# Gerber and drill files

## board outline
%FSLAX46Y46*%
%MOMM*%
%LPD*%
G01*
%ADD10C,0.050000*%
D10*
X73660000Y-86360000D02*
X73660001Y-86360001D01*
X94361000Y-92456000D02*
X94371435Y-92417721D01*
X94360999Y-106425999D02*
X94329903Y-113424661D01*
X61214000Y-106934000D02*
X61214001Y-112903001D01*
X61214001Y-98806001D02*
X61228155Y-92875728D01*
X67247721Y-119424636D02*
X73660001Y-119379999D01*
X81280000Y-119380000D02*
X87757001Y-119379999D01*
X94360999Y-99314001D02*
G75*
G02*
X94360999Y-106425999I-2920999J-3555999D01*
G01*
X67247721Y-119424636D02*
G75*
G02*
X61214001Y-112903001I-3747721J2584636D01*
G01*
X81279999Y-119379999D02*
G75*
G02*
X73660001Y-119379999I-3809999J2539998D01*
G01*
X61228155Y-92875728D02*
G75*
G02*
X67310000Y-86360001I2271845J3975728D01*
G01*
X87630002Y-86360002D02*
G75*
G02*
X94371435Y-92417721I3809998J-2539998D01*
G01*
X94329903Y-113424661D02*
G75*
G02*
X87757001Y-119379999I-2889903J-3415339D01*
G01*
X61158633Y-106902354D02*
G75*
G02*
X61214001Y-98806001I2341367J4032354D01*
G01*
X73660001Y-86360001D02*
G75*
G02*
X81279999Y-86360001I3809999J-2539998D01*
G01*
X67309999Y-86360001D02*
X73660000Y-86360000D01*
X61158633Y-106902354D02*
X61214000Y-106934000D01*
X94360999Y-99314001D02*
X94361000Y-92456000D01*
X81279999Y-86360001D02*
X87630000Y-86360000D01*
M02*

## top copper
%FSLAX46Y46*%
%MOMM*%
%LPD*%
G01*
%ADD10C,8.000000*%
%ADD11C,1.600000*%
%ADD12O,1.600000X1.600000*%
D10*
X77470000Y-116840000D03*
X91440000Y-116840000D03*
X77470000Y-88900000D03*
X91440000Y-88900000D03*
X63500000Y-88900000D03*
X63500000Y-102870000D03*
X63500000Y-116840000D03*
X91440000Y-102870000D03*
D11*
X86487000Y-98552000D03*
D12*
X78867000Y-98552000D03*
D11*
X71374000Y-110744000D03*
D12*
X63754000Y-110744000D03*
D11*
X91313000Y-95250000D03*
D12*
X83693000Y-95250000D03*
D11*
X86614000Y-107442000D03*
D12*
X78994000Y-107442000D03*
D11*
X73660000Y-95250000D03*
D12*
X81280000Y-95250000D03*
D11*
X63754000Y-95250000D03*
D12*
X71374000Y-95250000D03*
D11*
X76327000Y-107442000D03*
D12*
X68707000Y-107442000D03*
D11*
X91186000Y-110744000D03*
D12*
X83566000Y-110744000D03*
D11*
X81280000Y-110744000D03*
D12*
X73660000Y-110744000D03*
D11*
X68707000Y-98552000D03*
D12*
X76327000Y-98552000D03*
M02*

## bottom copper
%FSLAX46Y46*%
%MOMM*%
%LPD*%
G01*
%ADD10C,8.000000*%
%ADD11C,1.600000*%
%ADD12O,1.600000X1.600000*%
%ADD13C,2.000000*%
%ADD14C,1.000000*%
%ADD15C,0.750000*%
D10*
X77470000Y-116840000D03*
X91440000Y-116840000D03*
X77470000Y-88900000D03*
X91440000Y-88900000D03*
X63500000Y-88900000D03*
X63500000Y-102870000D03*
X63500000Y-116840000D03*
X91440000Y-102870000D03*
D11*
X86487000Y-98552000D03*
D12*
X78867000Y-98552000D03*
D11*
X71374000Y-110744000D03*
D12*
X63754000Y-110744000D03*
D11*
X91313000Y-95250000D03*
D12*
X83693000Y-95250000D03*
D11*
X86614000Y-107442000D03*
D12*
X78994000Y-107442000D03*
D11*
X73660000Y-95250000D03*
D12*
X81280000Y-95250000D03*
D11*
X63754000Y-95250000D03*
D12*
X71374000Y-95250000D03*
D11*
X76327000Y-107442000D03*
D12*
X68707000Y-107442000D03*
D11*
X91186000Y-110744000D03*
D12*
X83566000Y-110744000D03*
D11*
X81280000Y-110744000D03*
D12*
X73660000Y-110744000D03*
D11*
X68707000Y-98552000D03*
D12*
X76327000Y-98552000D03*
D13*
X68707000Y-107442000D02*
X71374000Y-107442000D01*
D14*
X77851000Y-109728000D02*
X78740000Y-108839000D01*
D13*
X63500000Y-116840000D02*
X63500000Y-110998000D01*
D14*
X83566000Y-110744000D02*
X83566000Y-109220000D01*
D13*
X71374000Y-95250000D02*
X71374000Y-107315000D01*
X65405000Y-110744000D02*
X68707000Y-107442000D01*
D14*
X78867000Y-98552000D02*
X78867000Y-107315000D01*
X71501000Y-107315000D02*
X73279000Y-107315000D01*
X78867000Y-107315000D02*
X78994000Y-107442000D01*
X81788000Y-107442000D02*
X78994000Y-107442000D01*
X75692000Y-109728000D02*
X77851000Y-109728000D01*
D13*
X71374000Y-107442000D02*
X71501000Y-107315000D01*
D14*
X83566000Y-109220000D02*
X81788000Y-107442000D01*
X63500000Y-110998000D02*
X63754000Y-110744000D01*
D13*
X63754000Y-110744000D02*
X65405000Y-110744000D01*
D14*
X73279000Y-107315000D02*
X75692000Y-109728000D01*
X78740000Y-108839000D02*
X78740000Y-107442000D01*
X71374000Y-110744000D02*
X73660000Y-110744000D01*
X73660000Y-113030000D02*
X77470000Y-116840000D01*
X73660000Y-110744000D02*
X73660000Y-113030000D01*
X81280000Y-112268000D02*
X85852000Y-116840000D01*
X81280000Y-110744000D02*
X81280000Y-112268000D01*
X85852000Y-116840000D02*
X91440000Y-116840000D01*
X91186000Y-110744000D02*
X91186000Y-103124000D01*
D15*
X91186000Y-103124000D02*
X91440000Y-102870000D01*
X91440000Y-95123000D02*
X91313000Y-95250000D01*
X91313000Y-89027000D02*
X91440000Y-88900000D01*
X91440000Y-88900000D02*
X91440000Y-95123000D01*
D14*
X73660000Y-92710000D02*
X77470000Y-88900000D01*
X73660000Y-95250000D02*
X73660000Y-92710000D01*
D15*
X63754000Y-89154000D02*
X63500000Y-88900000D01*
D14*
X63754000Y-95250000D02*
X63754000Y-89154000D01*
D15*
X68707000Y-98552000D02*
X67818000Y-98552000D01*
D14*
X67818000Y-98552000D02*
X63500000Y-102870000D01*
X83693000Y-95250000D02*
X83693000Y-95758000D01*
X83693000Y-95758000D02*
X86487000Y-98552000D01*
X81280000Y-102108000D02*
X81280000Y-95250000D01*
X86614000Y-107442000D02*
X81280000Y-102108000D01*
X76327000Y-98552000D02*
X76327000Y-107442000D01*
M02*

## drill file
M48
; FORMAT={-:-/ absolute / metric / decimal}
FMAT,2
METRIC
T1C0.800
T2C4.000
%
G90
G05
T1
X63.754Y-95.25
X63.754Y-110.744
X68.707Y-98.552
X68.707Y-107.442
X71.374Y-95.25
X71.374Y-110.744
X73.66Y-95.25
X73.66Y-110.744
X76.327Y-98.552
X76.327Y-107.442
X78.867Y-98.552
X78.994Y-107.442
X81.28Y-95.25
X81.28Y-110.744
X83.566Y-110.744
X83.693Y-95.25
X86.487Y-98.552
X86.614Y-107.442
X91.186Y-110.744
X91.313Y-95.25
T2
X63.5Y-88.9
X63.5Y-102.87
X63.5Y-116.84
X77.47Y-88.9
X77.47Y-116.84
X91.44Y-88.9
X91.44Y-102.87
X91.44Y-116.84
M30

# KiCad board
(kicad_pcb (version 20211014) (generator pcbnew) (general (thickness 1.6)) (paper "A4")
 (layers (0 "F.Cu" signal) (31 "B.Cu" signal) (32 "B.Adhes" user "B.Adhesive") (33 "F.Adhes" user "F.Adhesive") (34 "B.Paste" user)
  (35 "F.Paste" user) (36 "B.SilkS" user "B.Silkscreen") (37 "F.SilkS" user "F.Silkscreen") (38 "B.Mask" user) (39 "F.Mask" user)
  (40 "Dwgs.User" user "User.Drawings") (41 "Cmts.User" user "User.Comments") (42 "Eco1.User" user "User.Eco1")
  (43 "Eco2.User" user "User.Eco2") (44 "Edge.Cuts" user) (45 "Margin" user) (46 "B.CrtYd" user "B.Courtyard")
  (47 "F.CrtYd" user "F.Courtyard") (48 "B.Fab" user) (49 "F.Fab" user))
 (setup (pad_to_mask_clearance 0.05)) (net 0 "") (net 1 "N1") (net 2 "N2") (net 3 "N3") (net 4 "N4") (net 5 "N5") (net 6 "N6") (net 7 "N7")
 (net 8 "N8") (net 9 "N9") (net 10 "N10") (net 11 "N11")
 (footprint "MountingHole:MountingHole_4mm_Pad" (layer "F.Cu") (at 77.47 116.84)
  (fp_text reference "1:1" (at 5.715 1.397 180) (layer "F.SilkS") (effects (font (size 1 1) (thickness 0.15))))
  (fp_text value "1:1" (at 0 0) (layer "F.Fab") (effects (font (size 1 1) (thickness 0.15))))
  (pad "1" thru_hole circle locked (at 0 0) (size 8 8) (drill 4) (layers *.Cu *.Mask) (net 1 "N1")))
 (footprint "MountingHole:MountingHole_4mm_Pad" (layer "F.Cu") (at 91.44 116.84)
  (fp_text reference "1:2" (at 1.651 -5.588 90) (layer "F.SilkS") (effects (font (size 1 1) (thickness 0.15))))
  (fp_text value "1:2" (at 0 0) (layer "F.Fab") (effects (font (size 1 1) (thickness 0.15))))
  (pad "1" thru_hole circle locked (at 0 0) (size 8 8) (drill 4) (layers *.Cu *.Mask) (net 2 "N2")))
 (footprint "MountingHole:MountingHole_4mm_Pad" (layer "F.Cu") (at 77.47 88.9)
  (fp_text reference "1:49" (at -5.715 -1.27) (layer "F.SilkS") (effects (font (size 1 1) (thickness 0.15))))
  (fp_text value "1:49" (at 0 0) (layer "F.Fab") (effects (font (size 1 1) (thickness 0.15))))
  (pad "1" thru_hole circle locked (at 0 0) (size 8 8) (drill 4) (layers *.Cu *.Mask) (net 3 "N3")))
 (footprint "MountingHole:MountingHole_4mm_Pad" (layer "F.Cu") (at 91.44 88.9)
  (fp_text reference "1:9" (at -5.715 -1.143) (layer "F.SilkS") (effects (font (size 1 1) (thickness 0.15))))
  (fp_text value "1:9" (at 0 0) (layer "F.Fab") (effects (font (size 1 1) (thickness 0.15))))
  (pad "1" thru_hole circle locked (at 0 0) (size 8 8) (drill 4) (layers *.Cu *.Mask) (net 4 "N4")))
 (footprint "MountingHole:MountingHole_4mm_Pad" (layer "F.Cu") (at 63.5 88.9)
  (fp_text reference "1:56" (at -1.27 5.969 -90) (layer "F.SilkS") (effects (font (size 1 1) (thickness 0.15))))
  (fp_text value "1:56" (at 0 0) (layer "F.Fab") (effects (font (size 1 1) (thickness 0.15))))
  (pad "1" thru_hole circle locked (at 0 0) (size 8 8) (drill 4) (layers *.Cu *.Mask) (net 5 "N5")))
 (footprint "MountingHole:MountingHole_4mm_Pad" (layer "F.Cu") (at 63.5 102.87)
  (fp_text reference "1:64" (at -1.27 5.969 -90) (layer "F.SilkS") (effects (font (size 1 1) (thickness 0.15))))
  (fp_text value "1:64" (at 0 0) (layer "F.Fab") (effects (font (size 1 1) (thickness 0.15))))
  (pad "1" thru_hole circle locked (at 0 0) (size 8 8) (drill 4) (layers *.Cu *.Mask) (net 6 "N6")))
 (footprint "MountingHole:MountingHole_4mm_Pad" (layer "F.Cu") (at 63.5 116.84)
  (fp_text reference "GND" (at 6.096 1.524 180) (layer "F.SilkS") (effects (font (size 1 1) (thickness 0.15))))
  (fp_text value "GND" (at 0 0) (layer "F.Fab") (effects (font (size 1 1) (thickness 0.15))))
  (pad "1" thru_hole circle locked (at 0 0) (size 8 8) (drill 4) (layers *.Cu *.Mask) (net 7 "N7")))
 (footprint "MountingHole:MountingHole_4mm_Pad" (layer "F.Cu") (at 91.44 102.87)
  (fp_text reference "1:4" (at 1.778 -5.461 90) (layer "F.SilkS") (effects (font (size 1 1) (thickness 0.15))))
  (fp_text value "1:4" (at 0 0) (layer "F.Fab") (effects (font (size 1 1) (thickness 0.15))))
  (pad "1" thru_hole circle locked (at 0 0) (size 8 8) (drill 4) (layers *.Cu *.Mask) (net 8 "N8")))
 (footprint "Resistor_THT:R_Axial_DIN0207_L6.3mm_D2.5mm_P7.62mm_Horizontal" (layer "F.Cu") (at 86.487 98.552 180)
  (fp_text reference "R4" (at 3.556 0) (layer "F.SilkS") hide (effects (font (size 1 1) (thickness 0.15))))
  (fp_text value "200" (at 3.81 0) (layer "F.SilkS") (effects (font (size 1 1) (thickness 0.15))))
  (pad "1" thru_hole circle locked (at 0 0 180) (size 1.6 1.6) (drill 0.8) (layers *.Cu *.Mask) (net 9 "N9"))
  (pad "2" thru_hole oval locked (at 7.62 0 180) (size 1.6 1.6) (drill 0.8) (layers *.Cu *.Mask) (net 7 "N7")))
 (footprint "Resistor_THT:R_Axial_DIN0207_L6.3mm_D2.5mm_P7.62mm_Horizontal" (layer "F.Cu") (at 71.374 110.744 180)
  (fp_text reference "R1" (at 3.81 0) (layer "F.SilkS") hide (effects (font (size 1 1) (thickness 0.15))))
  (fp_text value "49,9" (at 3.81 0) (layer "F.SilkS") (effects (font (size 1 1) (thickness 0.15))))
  (pad "1" thru_hole circle locked (at 0 0 180) (size 1.6 1.6) (drill 0.8) (layers *.Cu *.Mask) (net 1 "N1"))
  (pad "2" thru_hole oval locked (at 7.62 0 180) (size 1.6 1.6) (drill 0.8) (layers *.Cu *.Mask) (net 7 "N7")))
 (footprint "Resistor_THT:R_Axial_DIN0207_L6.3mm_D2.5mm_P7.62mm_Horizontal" (layer "F.Cu") (at 91.313 95.25 180)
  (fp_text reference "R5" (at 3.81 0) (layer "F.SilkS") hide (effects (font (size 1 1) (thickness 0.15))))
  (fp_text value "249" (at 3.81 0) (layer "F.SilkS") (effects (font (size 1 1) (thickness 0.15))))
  (pad "1" thru_hole circle locked (at 0 0 180) (size 1.6 1.6) (drill 0.8) (layers *.Cu *.Mask) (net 4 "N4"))
  (pad "2" thru_hole oval locked (at 7.62 0 180) (size 1.6 1.6) (drill 0.8) (layers *.Cu *.Mask) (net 9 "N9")))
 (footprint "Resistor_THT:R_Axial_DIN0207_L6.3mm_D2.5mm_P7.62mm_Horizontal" (layer "F.Cu") (at 86.614 107.442 180)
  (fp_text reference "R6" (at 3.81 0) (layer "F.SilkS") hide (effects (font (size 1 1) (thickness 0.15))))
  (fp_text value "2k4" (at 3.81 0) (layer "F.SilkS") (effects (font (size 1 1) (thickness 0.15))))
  (pad "1" thru_hole circle locked (at 0 0 180) (size 1.6 1.6) (drill 0.8) (layers *.Cu *.Mask) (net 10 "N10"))
  (pad "2" thru_hole oval locked (at 7.62 0 180) (size 1.6 1.6) (drill 0.8) (layers *.Cu *.Mask) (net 7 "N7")))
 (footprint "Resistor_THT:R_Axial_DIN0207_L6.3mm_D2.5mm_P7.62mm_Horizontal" (layer "F.Cu") (at 73.66 95.25)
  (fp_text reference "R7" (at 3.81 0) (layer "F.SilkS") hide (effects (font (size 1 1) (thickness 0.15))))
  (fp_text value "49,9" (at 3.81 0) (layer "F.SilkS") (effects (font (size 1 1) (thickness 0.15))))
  (pad "1" thru_hole circle locked (at 0 0) (size 1.6 1.6) (drill 0.8) (layers *.Cu *.Mask) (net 3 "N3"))
  (pad "2" thru_hole oval locked (at 7.62 0) (size 1.6 1.6) (drill 0.8) (layers *.Cu *.Mask) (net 10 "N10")))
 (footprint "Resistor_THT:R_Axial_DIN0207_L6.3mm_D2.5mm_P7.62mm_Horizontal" (layer "F.Cu") (at 63.754 95.25)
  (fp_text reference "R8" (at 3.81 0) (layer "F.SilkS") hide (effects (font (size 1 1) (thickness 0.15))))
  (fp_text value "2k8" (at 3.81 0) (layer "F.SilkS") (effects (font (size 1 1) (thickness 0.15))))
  (pad "1" thru_hole circle locked (at 0 0) (size 1.6 1.6) (drill 0.8) (layers *.Cu *.Mask) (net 5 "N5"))
  (pad "2" thru_hole oval locked (at 7.62 0) (size 1.6 1.6) (drill 0.8) (layers *.Cu *.Mask) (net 7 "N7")))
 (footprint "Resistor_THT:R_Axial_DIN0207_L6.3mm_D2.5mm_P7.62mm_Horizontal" (layer "F.Cu") (at 76.327 107.442 180)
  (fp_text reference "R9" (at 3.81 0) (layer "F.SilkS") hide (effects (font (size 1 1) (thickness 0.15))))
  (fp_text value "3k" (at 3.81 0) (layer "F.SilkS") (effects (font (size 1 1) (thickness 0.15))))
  (pad "1" thru_hole circle locked (at 0 0 180) (size 1.6 1.6) (drill 0.8) (layers *.Cu *.Mask) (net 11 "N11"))
  (pad "2" thru_hole oval locked (at 7.62 0 180) (size 1.6 1.6) (drill 0.8) (layers *.Cu *.Mask) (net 7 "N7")))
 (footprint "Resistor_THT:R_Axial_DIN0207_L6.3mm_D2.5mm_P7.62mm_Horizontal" (layer "F.Cu") (at 91.186 110.744 180)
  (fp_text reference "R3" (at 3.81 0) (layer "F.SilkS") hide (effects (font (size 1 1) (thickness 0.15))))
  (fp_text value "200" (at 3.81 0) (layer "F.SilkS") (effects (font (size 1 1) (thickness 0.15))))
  (pad "1" thru_hole circle locked (at 0 0 180) (size 1.6 1.6) (drill 0.8) (layers *.Cu *.Mask) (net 8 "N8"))
  (pad "2" thru_hole oval locked (at 7.62 0 180) (size 1.6 1.6) (drill 0.8) (layers *.Cu *.Mask) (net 7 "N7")))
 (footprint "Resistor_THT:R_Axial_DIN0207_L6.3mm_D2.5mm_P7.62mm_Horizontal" (layer "F.Cu") (at 81.28 110.744 180)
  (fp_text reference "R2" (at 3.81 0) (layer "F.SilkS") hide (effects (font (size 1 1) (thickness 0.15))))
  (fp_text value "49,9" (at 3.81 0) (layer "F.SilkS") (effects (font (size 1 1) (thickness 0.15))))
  (pad "1" thru_hole circle locked (at 0 0 180) (size 1.6 1.6) (drill 0.8) (layers *.Cu *.Mask) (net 2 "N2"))
  (pad "2" thru_hole oval locked (at 7.62 0 180) (size 1.6 1.6) (drill 0.8) (layers *.Cu *.Mask) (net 1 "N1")))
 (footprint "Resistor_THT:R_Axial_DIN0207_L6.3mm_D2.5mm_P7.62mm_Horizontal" (layer "F.Cu") (at 68.707 98.552)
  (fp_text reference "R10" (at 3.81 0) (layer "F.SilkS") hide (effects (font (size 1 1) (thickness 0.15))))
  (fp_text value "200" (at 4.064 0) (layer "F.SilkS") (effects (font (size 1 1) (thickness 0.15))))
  (pad "1" thru_hole circle locked (at 0 0) (size 1.6 1.6) (drill 0.8) (layers *.Cu *.Mask) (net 6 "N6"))
  (pad "2" thru_hole oval locked (at 7.62 0) (size 1.6 1.6) (drill 0.8) (layers *.Cu *.Mask) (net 11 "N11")))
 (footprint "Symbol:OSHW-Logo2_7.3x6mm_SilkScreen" (layer "F.Cu") (at 72.39 102.87)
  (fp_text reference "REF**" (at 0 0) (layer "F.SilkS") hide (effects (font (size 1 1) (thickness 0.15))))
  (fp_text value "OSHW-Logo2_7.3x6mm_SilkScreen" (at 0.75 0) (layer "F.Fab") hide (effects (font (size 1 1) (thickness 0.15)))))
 (gr_line (start 73.66 86.36) (end 73.660001 86.360001) (layer "Edge.Cuts") (width 0.05))
 (gr_line (start 94.361 92.456) (end 94.371435 92.417721) (layer "Edge.Cuts") (width 0.05))
 (gr_line (start 94.360999 106.425999) (end 94.329903 113.424661) (layer "Edge.Cuts") (width 0.05))
 (gr_line (start 61.214 106.934) (end 61.214001 112.903001) (layer "Edge.Cuts") (width 0.05))
 (gr_line (start 61.214001 98.806001) (end 61.228155 92.875728) (layer "Edge.Cuts") (width 0.05))
 (gr_line (start 67.247721 119.424636) (end 73.660001 119.379999) (layer "Edge.Cuts") (width 0.05))
 (gr_line (start 81.28 119.38) (end 87.757001 119.379999) (layer "Edge.Cuts") (width 0.05))
 (gr_arc (start 94.360999 99.314001) (mid 96.041887 102.87) (end 94.360999 106.425999) (layer "Edge.Cuts") (width 0.05))
 (gr_arc (start 67.247721 119.424636) (mid 60.15828 119.931709) (end 61.214001 112.903001) (layer "Edge.Cuts") (width 0.05))
 (gr_arc (start 81.279999 119.379999) (mid 77.47 121.419049) (end 73.660001 119.379999) (layer "Edge.Cuts") (width 0.05))
 (gr_arc (start 61.228155 92.875728) (mid 60.15259 85.775494) (end 67.309999 86.360001) (layer "Edge.Cuts") (width 0.05))
 (gr_arc (start 87.630002 86.360002) (mid 94.500549 85.494018) (end 94.371435 92.417721) (layer "Edge.Cuts") (width 0.05))
 (gr_arc (start 94.329903 113.424661) (mid 94.443958 120.155466) (end 87.757001 119.379999) (layer "Edge.Cuts") (width 0.05))
 (gr_arc (start 61.158633 106.902354) (mid 58.83729 102.838113) (end 61.214001 98.806001) (layer "Edge.Cuts") (width 0.05))
 (gr_arc (start 73.660001 86.360001) (mid 77.47 84.320951) (end 81.279999 86.360001) (layer "Edge.Cuts") (width 0.05))
 (gr_line (start 67.309999 86.360001) (end 73.66 86.36) (layer "Edge.Cuts") (width 0.05))
 (gr_line (start 61.158633 106.902354) (end 61.214 106.934) (layer "Edge.Cuts") (width 0.05))
 (gr_line (start 94.360999 99.314001) (end 94.361 92.456) (layer "Edge.Cuts") (width 0.05))
 (gr_line (start 81.279999 86.360001) (end 87.63 86.36) (layer "Edge.Cuts") (width 0.05))
 (segment (start 68.707 107.442) (end 71.374 107.442) (width 2) (layer "B.Cu") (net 7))
 (segment (start 77.851 109.728) (end 78.74 108.839) (width 1) (layer "B.Cu") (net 7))
 (segment (start 63.5 116.84) (end 63.5 110.998) (width 2) (layer "B.Cu") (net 7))
 (segment (start 83.566 110.744) (end 83.566 109.22) (width 1) (layer "B.Cu") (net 7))
 (segment (start 71.374 95.25) (end 71.374 107.315) (width 2) (layer "B.Cu") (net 7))
 (segment (start 65.405 110.744) (end 68.707 107.442) (width 2) (layer "B.Cu") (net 7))
 (segment (start 78.867 98.552) (end 78.867 107.315) (width 1) (layer "B.Cu") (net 7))
 (segment (start 71.501 107.315) (end 73.279 107.315) (width 1) (layer "B.Cu") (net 7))
 (segment (start 78.867 107.315) (end 78.994 107.442) (width 1) (layer "B.Cu") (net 7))
 (segment (start 81.788 107.442) (end 78.994 107.442) (width 1) (layer "B.Cu") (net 7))
 (segment (start 75.692 109.728) (end 77.851 109.728) (width 1) (layer "B.Cu") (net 7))
 (segment (start 71.374 107.442) (end 71.501 107.315) (width 2) (layer "B.Cu") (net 7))
 (segment (start 83.566 109.22) (end 81.788 107.442) (width 1) (layer "B.Cu") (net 7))
 (segment (start 63.5 110.998) (end 63.754 110.744) (width 1) (layer "B.Cu") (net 7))
 (segment (start 63.754 110.744) (end 65.405 110.744) (width 2) (layer "B.Cu") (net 7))
 (segment (start 73.279 107.315) (end 75.692 109.728) (width 1) (layer "B.Cu") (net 7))
 (segment (start 78.74 108.839) (end 78.74 107.442) (width 1) (layer "B.Cu") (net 7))
 (segment (start 71.374 110.744) (end 73.66 110.744) (width 1) (layer "B.Cu") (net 1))
 (segment (start 73.66 113.03) (end 77.47 116.84) (width 1) (layer "B.Cu") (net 1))
 (segment (start 73.66 110.744) (end 73.66 113.03) (width 1) (layer "B.Cu") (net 1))
 (segment (start 81.28 112.268) (end 85.852 116.84) (width 1) (layer "B.Cu") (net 2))
 (segment (start 81.28 110.744) (end 81.28 112.268) (width 1) (layer "B.Cu") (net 2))
 (segment (start 85.852 116.84) (end 91.44 116.84) (width 1) (layer "B.Cu") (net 2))
 (segment (start 91.186 110.744) (end 91.186 103.124) (width 1) (layer "B.Cu") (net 8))
 (segment (start 91.186 103.124) (end 91.44 102.87) (width 0.75) (layer "B.Cu") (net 8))
 (segment (start 91.44 95.123) (end 91.313 95.25) (width 0.75) (layer "B.Cu") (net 4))
 (segment (start 91.313 89.027) (end 91.44 88.9) (width 0.75) (layer "B.Cu") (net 4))
 (segment (start 91.44 88.9) (end 91.44 95.123) (width 0.75) (layer "B.Cu") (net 4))
 (segment (start 73.66 92.71) (end 77.47 88.9) (width 1) (layer "B.Cu") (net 3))
 (segment (start 73.66 95.25) (end 73.66 92.71) (width 1) (layer "B.Cu") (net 3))
 (segment (start 63.754 89.154) (end 63.5 88.9) (width 0.75) (layer "B.Cu") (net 5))
 (segment (start 63.754 95.25) (end 63.754 89.154) (width 1) (layer "B.Cu") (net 5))
 (segment (start 68.707 98.552) (end 67.818 98.552) (width 0.75) (layer "B.Cu") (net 6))
 (segment (start 67.818 98.552) (end 63.5 102.87) (width 1) (layer "B.Cu") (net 6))
 (segment (start 83.693 95.25) (end 83.693 95.758) (width 1) (layer "B.Cu") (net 9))
 (segment (start 83.693 95.758) (end 86.487 98.552) (width 1) (layer "B.Cu") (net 9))
 (segment (start 81.28 102.108) (end 81.28 95.25) (width 1) (layer "B.Cu") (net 10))
 (segment (start 86.614 107.442) (end 81.28 102.108) (width 1) (layer "B.Cu") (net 10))
 (segment (start 76.327 98.552) (end 76.327 107.442) (width 1) (layer "B.Cu") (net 11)))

